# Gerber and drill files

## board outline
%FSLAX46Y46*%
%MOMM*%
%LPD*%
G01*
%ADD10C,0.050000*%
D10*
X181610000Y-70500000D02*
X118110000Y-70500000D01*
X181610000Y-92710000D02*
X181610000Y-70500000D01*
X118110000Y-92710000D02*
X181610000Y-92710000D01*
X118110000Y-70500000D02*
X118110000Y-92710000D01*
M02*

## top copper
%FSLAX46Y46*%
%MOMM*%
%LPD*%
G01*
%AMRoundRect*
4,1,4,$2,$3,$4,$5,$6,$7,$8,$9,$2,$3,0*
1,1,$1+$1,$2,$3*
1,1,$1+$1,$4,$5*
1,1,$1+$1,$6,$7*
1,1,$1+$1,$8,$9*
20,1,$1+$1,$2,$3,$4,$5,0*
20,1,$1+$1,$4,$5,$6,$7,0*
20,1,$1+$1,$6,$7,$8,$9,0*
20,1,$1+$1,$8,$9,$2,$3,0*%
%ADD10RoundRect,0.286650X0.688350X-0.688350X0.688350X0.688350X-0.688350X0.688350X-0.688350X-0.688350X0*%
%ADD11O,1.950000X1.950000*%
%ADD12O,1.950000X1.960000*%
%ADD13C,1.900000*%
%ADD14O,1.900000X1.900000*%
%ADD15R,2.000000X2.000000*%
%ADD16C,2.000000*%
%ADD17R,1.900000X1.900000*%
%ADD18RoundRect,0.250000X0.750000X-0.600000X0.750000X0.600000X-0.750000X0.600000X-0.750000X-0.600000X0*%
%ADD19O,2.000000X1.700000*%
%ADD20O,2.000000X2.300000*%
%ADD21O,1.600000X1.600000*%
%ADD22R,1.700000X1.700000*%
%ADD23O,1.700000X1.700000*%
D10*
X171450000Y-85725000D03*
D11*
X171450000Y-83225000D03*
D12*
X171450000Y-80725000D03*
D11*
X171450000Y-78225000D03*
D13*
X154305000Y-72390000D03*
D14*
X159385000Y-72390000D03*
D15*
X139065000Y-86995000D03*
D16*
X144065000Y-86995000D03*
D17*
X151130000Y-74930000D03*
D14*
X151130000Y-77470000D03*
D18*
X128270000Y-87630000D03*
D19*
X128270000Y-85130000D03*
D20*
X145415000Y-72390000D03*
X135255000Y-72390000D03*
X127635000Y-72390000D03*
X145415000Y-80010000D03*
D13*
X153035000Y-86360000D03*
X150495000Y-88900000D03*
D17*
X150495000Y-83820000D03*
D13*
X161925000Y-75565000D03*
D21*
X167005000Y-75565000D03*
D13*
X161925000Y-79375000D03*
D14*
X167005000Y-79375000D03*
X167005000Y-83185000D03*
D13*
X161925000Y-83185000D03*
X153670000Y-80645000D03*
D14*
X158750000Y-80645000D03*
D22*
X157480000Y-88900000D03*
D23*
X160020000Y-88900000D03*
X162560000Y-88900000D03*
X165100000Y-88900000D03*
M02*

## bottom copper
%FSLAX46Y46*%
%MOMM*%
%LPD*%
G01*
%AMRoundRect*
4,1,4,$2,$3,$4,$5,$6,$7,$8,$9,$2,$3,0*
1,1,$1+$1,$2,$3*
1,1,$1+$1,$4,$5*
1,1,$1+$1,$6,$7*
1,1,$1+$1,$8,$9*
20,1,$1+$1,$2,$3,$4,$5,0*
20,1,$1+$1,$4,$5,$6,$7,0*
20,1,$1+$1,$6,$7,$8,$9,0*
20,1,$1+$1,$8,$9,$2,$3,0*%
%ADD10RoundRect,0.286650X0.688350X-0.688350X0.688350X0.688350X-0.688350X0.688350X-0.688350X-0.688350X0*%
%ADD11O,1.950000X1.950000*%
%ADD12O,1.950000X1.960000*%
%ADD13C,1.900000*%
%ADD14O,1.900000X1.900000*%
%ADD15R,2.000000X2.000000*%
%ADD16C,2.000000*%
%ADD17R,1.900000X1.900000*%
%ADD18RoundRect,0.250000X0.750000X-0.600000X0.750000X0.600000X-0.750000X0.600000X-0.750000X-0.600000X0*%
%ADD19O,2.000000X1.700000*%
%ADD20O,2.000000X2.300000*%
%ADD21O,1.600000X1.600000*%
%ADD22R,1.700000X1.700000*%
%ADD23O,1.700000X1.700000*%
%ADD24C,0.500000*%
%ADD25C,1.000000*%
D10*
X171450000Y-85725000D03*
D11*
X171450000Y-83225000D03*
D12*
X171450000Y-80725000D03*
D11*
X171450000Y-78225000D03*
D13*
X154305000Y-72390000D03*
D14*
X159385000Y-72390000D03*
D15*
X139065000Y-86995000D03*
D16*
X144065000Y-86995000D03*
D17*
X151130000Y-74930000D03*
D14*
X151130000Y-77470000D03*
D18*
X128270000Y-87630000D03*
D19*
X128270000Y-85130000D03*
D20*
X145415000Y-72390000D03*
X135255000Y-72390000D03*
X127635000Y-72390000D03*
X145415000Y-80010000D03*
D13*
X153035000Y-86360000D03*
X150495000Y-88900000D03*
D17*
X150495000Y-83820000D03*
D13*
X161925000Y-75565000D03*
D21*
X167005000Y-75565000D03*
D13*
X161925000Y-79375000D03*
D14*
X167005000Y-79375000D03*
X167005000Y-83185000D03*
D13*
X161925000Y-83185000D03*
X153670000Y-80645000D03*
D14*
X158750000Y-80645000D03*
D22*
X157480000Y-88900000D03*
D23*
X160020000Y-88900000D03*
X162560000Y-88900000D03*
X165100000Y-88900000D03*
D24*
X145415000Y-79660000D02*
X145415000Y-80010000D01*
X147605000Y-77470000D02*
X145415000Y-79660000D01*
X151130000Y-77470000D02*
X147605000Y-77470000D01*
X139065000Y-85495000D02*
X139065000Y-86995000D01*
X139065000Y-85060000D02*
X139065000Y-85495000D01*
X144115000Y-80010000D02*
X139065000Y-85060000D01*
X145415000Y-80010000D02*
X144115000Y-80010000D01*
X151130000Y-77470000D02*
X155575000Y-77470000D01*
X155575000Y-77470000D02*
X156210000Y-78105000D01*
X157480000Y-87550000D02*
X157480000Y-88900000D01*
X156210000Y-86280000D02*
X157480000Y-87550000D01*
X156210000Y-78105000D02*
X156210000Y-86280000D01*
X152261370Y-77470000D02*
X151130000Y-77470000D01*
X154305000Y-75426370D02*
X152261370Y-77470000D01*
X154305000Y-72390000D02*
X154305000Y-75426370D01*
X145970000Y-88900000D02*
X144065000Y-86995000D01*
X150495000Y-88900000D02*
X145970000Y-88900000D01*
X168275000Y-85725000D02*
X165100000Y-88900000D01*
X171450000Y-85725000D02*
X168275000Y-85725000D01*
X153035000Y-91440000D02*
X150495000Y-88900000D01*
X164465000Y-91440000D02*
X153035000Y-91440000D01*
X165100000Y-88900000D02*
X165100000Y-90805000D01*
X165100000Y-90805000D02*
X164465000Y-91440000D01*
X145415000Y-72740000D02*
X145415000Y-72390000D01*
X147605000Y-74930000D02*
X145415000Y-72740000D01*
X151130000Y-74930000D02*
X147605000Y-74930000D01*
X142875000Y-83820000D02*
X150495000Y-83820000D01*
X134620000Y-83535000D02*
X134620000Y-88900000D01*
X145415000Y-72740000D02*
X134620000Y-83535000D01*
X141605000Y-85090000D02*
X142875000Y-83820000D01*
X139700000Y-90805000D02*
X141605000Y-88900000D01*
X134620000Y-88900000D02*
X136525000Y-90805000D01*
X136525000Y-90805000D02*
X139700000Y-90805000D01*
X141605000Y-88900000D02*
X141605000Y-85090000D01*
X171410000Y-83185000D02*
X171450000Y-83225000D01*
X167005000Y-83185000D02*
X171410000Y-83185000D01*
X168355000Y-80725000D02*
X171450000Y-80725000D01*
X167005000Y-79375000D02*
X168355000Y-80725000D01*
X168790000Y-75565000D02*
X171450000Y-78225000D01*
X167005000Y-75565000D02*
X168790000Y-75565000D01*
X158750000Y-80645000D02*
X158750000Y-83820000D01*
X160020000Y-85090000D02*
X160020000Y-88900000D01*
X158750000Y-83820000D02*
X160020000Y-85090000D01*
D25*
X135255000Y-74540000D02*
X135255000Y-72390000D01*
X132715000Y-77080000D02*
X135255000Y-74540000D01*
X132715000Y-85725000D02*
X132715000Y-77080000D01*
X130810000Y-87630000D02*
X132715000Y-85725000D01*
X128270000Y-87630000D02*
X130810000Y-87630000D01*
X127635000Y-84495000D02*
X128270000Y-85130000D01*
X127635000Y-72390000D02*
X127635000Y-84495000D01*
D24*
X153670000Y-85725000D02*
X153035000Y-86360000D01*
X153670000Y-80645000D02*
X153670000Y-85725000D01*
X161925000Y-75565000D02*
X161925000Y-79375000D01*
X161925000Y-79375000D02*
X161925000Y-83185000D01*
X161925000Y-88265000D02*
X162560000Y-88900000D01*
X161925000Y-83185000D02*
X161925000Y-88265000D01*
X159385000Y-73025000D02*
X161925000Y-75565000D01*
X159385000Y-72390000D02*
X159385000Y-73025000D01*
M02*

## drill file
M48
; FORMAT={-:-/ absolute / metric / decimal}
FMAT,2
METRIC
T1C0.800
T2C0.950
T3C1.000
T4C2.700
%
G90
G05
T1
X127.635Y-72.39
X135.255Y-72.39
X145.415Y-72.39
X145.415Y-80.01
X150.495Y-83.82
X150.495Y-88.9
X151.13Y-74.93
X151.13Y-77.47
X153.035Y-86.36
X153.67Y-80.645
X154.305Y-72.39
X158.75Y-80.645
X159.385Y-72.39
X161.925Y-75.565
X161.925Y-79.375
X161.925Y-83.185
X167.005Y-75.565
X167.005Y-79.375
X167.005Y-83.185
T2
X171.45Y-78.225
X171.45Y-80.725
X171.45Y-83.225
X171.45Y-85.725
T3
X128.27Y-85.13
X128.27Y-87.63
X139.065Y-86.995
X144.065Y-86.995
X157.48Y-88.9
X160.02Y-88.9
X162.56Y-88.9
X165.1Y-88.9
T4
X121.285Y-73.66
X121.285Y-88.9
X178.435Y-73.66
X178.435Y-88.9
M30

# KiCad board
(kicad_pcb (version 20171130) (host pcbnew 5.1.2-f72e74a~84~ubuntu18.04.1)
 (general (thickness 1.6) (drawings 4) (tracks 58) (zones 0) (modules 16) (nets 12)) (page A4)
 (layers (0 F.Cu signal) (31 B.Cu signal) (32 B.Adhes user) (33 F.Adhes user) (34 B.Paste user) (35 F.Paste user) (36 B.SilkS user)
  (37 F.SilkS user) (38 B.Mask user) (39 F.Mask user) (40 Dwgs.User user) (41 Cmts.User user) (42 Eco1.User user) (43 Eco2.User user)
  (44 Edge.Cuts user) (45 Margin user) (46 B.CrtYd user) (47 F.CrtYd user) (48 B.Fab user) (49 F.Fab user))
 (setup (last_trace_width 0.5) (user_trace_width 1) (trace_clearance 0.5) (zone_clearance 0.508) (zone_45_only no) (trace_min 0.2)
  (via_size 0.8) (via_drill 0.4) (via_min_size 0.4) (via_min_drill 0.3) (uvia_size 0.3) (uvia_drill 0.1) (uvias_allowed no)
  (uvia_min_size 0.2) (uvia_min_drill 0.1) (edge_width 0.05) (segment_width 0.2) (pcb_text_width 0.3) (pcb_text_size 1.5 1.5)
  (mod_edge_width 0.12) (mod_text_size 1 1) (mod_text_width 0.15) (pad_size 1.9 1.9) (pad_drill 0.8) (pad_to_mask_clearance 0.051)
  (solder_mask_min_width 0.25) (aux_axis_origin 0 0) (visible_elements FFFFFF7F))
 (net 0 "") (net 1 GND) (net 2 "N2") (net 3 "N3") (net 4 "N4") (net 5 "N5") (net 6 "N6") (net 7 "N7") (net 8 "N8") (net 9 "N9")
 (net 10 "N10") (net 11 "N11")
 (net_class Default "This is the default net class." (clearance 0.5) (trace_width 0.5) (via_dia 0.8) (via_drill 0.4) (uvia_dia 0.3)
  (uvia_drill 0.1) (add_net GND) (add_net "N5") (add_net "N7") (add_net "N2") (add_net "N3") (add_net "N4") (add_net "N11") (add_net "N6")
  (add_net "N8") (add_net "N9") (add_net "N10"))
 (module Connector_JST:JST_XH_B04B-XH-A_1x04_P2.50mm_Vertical (layer F.Cu) (at 171.45 85.725 90)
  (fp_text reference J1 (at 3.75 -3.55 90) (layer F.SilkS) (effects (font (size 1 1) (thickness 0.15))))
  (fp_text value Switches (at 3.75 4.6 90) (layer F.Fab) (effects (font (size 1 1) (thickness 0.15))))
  (pad 1 thru_hole roundrect (at 0 0 90) (size 1.95 1.95) (drill 0.95) (layers *.Cu *.Mask) (roundrect_rratio 0.147) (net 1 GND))
  (pad 2 thru_hole oval (at 2.5 0 90) (size 1.95 1.95) (drill 0.95) (layers *.Cu *.Mask) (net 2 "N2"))
  (pad 3 thru_hole oval (at 5 0 90) (size 1.96 1.95) (drill 0.95) (layers *.Cu *.Mask) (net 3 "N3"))
  (pad 4 thru_hole oval (at 7.5 0 90) (size 1.95 1.95) (drill 0.95) (layers *.Cu *.Mask) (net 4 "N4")))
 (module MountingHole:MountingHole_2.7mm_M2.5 (layer F.Cu) (at 121.285 73.66)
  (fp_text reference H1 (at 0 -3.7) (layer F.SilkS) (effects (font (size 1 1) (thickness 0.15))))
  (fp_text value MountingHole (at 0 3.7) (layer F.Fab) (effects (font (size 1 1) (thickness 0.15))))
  (pad 1 np_thru_hole circle (at 0 0) (size 2.7 2.7) (drill 2.7) (layers *.Cu *.Mask)))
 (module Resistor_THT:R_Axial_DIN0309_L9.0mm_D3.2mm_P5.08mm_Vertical (layer F.Cu) (at 154.305 72.39)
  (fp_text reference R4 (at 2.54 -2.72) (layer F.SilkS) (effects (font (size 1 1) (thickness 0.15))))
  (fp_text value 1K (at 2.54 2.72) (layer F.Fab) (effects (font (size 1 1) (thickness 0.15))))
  (pad 1 thru_hole circle (at 0 0) (size 1.9 1.9) (drill 0.8) (layers *.Cu *.Mask) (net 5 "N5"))
  (pad 2 thru_hole oval (at 5.08 0) (size 1.9 1.9) (drill 0.8) (layers *.Cu *.Mask) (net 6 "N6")))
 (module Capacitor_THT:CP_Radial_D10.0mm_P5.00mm (layer F.Cu) (at 139.065 86.995)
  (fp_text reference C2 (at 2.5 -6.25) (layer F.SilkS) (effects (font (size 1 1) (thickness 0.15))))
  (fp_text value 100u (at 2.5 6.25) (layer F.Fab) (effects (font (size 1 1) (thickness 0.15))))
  (pad 1 thru_hole rect (at 0 0) (size 2 2) (drill 1) (layers *.Cu *.Mask) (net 5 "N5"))
  (pad 2 thru_hole circle (at 5 0) (size 2 2) (drill 1) (layers *.Cu *.Mask) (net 1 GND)))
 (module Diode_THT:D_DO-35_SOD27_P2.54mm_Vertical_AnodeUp (layer F.Cu) (at 151.13 74.93 270)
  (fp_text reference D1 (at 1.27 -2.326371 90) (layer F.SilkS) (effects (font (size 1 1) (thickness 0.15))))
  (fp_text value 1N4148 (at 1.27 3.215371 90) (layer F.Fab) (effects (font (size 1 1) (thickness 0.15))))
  (pad 1 thru_hole rect (at 0 0 270) (size 1.9 1.9) (drill 0.8) (layers *.Cu *.Mask) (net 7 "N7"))
  (pad 2 thru_hole oval (at 2.54 0 270) (size 1.9 1.9) (drill 0.8) (layers *.Cu *.Mask) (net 5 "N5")))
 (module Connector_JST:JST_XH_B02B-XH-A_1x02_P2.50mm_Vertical (layer F.Cu) (at 128.27 87.63 90)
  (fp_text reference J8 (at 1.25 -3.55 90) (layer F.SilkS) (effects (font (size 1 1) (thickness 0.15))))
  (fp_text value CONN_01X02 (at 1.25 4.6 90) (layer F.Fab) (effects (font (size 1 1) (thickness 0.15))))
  (pad 1 thru_hole roundrect (at 0 0 90) (size 1.7 2) (drill 1) (layers *.Cu *.Mask) (roundrect_rratio 0.147059) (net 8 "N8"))
  (pad 2 thru_hole oval (at 2.5 0 90) (size 1.7 2) (drill 1) (layers *.Cu *.Mask) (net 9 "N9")))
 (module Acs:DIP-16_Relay (layer F.Cu) (at 145.415 72.39 270)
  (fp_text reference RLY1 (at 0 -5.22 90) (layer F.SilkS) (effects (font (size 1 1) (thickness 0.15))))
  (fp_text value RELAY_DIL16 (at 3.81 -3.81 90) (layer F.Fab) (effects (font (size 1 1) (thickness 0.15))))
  (pad 1 thru_hole oval (at 0 0 270) (size 2.3 2) (drill 0.8) (layers *.Cu *.Mask F.SilkS) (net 7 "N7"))
  (pad 5 thru_hole oval (at 0 10.16 270) (size 2.3 2) (drill 0.8) (layers *.Cu *.Mask F.SilkS) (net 8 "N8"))
  (pad 8 thru_hole oval (at 0 17.78 270) (size 2.3 2) (drill 0.8) (layers *.Cu *.Mask F.SilkS) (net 9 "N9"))
  (pad 16 thru_hole oval (at 7.62 0 270) (size 2.3 2) (drill 0.8) (layers *.Cu *.Mask F.SilkS) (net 5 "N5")))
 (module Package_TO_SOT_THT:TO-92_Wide (layer F.Cu) (at 150.495 83.82 270)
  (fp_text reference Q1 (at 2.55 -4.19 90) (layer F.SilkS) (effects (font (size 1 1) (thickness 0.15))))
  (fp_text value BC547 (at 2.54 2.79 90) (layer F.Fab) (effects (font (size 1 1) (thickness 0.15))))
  (pad 2 thru_hole circle (at 2.54 -2.54) (size 1.9 1.9) (drill 0.8) (layers *.Cu *.Mask) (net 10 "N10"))
  (pad 3 thru_hole circle (at 5.08 0) (size 1.9 1.9) (drill 0.8) (layers *.Cu *.Mask) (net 1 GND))
  (pad 1 thru_hole rect (at 0 0) (size 1.9 1.9) (drill 0.8) (layers *.Cu *.Mask) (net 7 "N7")))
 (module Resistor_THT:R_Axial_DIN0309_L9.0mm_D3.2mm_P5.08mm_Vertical (layer F.Cu) (at 161.925 75.565)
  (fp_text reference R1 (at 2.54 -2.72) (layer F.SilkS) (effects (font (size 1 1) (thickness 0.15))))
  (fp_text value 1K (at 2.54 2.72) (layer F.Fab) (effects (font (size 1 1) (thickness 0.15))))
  (pad 1 thru_hole circle (at 0 0) (size 1.9 1.9) (drill 0.8) (layers *.Cu *.Mask) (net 6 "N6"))
  (pad 2 thru_hole oval (at 5.08 0) (size 1.6 1.6) (drill 0.8) (layers *.Cu *.Mask) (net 4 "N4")))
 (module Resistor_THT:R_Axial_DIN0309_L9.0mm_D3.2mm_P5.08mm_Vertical (layer F.Cu) (at 161.925 79.375)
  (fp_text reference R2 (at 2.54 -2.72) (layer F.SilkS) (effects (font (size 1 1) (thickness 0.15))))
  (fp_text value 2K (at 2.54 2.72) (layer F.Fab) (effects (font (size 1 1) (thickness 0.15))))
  (pad 1 thru_hole circle (at 0 0) (size 1.9 1.9) (drill 0.8) (layers *.Cu *.Mask) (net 6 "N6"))
  (pad 2 thru_hole oval (at 5.08 0) (size 1.9 1.9) (drill 0.8) (layers *.Cu *.Mask) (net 3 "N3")))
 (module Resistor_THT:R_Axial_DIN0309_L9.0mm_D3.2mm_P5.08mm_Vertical (layer F.Cu) (at 161.925 83.185)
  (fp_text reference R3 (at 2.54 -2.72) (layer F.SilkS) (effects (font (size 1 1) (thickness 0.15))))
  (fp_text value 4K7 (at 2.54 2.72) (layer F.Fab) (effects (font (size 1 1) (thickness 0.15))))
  (pad 2 thru_hole oval (at 5.08 0) (size 1.9 1.9) (drill 0.8) (layers *.Cu *.Mask) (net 2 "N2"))
  (pad 1 thru_hole circle (at 0 0) (size 1.9 1.9) (drill 0.8) (layers *.Cu *.Mask) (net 6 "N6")))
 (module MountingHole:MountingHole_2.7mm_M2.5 (layer F.Cu) (at 121.285 88.9)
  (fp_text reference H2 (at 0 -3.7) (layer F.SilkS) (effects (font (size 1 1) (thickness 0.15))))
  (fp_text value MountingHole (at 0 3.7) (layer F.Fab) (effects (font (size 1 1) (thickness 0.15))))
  (pad 1 np_thru_hole circle (at 0 0) (size 2.7 2.7) (drill 2.7) (layers *.Cu *.Mask)))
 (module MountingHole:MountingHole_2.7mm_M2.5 (layer F.Cu) (at 178.435 73.66)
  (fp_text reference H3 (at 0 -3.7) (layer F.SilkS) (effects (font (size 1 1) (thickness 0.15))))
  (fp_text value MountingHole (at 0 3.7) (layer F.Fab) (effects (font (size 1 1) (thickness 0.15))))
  (pad 1 np_thru_hole circle (at 0 0) (size 2.7 2.7) (drill 2.7) (layers *.Cu *.Mask)))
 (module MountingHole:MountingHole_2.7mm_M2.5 (layer F.Cu) (at 178.435 88.9)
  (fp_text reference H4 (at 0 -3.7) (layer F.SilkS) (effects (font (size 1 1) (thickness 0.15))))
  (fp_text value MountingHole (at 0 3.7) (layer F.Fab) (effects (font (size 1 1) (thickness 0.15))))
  (pad 1 np_thru_hole circle (at 0 0) (size 2.7 2.7) (drill 2.7) (layers *.Cu *.Mask)))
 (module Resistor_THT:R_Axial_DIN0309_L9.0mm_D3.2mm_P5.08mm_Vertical (layer F.Cu) (at 153.67 80.645)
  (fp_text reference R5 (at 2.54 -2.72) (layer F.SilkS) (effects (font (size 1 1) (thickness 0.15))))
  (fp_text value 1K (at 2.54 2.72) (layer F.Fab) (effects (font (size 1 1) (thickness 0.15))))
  (pad 1 thru_hole circle (at 0 0) (size 1.9 1.9) (drill 0.8) (layers *.Cu *.Mask) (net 10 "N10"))
  (pad 2 thru_hole oval (at 5.08 0) (size 1.9 1.9) (drill 0.8) (layers *.Cu *.Mask) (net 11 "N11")))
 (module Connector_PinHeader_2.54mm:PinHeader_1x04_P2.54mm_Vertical (layer F.Cu) (at 157.48 88.9 90)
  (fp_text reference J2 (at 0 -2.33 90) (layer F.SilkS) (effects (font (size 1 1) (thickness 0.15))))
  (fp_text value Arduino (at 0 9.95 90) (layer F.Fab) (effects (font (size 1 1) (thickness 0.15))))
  (pad 1 thru_hole rect (at 0 0 90) (size 1.7 1.7) (drill 1) (layers *.Cu *.Mask) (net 5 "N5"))
  (pad 2 thru_hole oval (at 0 2.54 90) (size 1.7 1.7) (drill 1) (layers *.Cu *.Mask) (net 11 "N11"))
  (pad 3 thru_hole oval (at 0 5.08 90) (size 1.7 1.7) (drill 1) (layers *.Cu *.Mask) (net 6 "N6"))
  (pad 4 thru_hole oval (at 0 7.62 90) (size 1.7 1.7) (drill 1) (layers *.Cu *.Mask) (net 1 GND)))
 (gr_line (start 181.61 70.5) (end 118.11 70.5) (layer Edge.Cuts) (width 0.05))
 (gr_line (start 181.61 92.71) (end 181.61 70.5) (layer Edge.Cuts) (width 0.05))
 (gr_line (start 118.11 92.71) (end 181.61 92.71) (layer Edge.Cuts) (width 0.05))
 (gr_line (start 118.11 70.5) (end 118.11 92.71) (layer Edge.Cuts) (width 0.05))
 (segment (start 145.415 79.66) (end 145.415 80.01) (width 0.5) (layer B.Cu) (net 5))
 (segment (start 147.605 77.47) (end 145.415 79.66) (width 0.5) (layer B.Cu) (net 5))
 (segment (start 151.13 77.47) (end 147.605 77.47) (width 0.5) (layer B.Cu) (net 5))
 (segment (start 139.065 85.495) (end 139.065 86.995) (width 0.5) (layer B.Cu) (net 5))
 (segment (start 139.065 85.06) (end 139.065 85.495) (width 0.5) (layer B.Cu) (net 5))
 (segment (start 144.115 80.01) (end 139.065 85.06) (width 0.5) (layer B.Cu) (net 5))
 (segment (start 145.415 80.01) (end 144.115 80.01) (width 0.5) (layer B.Cu) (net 5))
 (segment (start 151.13 77.47) (end 155.575 77.47) (width 0.5) (layer B.Cu) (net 5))
 (segment (start 155.575 77.47) (end 156.21 78.105) (width 0.5) (layer B.Cu) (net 5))
 (segment (start 157.48 87.55) (end 157.48 88.9) (width 0.5) (layer B.Cu) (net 5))
 (segment (start 156.21 86.28) (end 157.48 87.55) (width 0.5) (layer B.Cu) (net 5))
 (segment (start 156.21 78.105) (end 156.21 86.28) (width 0.5) (layer B.Cu) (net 5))
 (segment (start 152.26137 77.47) (end 151.13 77.47) (width 0.5) (layer B.Cu) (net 5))
 (segment (start 154.305 75.42637) (end 152.26137 77.47) (width 0.5) (layer B.Cu) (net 5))
 (segment (start 154.305 72.39) (end 154.305 75.42637) (width 0.5) (layer B.Cu) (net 5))
 (segment (start 145.97 88.9) (end 144.065 86.995) (width 0.5) (layer B.Cu) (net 1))
 (segment (start 150.495 88.9) (end 145.97 88.9) (width 0.5) (layer B.Cu) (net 1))
 (segment (start 168.275 85.725) (end 165.1 88.9) (width 0.5) (layer B.Cu) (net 1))
 (segment (start 171.45 85.725) (end 168.275 85.725) (width 0.5) (layer B.Cu) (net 1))
 (segment (start 153.035 91.44) (end 150.495 88.9) (width 0.5) (layer B.Cu) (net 1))
 (segment (start 164.465 91.44) (end 153.035 91.44) (width 0.5) (layer B.Cu) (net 1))
 (segment (start 165.1 88.9) (end 165.1 90.805) (width 0.5) (layer B.Cu) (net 1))
 (segment (start 165.1 90.805) (end 164.465 91.44) (width 0.5) (layer B.Cu) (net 1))
 (segment (start 145.415 72.74) (end 145.415 72.39) (width 0.5) (layer B.Cu) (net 7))
 (segment (start 147.605 74.93) (end 145.415 72.74) (width 0.5) (layer B.Cu) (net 7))
 (segment (start 151.13 74.93) (end 147.605 74.93) (width 0.5) (layer B.Cu) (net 7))
 (segment (start 142.875 83.82) (end 150.495 83.82) (width 0.5) (layer B.Cu) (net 7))
 (segment (start 134.62 83.535) (end 134.62 88.9) (width 0.5) (layer B.Cu) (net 7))
 (segment (start 145.415 72.74) (end 134.62 83.535) (width 0.5) (layer B.Cu) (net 7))
 (segment (start 141.605 85.09) (end 142.875 83.82) (width 0.5) (layer B.Cu) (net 7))
 (segment (start 139.7 90.805) (end 141.605 88.9) (width 0.5) (layer B.Cu) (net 7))
 (segment (start 134.62 88.9) (end 136.525 90.805) (width 0.5) (layer B.Cu) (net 7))
 (segment (start 136.525 90.805) (end 139.7 90.805) (width 0.5) (layer B.Cu) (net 7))
 (segment (start 141.605 88.9) (end 141.605 85.09) (width 0.5) (layer B.Cu) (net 7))
 (segment (start 171.41 83.185) (end 171.45 83.225) (width 0.5) (layer B.Cu) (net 2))
 (segment (start 167.005 83.185) (end 171.41 83.185) (width 0.5) (layer B.Cu) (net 2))
 (segment (start 168.355 80.725) (end 171.45 80.725) (width 0.5) (layer B.Cu) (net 3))
 (segment (start 167.005 79.375) (end 168.355 80.725) (width 0.5) (layer B.Cu) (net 3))
 (segment (start 168.79 75.565) (end 171.45 78.225) (width 0.5) (layer B.Cu) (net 4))
 (segment (start 167.005 75.565) (end 168.79 75.565) (width 0.5) (layer B.Cu) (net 4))
 (segment (start 158.75 80.645) (end 158.75 83.82) (width 0.5) (layer B.Cu) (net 11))
 (segment (start 160.02 85.09) (end 160.02 88.9) (width 0.5) (layer B.Cu) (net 11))
 (segment (start 158.75 83.82) (end 160.02 85.09) (width 0.5) (layer B.Cu) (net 11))
 (segment (start 135.255 74.54) (end 135.255 72.39) (width 1) (layer B.Cu) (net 8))
 (segment (start 132.715 77.08) (end 135.255 74.54) (width 1) (layer B.Cu) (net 8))
 (segment (start 132.715 85.725) (end 132.715 77.08) (width 1) (layer B.Cu) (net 8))
 (segment (start 130.81 87.63) (end 132.715 85.725) (width 1) (layer B.Cu) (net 8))
 (segment (start 128.27 87.63) (end 130.81 87.63) (width 1) (layer B.Cu) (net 8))
 (segment (start 127.635 84.495) (end 128.27 85.13) (width 1) (layer B.Cu) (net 9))
 (segment (start 127.635 72.39) (end 127.635 84.495) (width 1) (layer B.Cu) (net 9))
 (segment (start 153.67 85.725) (end 153.035 86.36) (width 0.5) (layer B.Cu) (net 10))
 (segment (start 153.67 80.645) (end 153.67 85.725) (width 0.5) (layer B.Cu) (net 10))
 (segment (start 161.925 75.565) (end 161.925 79.375) (width 0.5) (layer B.Cu) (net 6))
 (segment (start 161.925 79.375) (end 161.925 83.185) (width 0.5) (layer B.Cu) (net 6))
 (segment (start 161.925 88.265) (end 162.56 88.9) (width 0.5) (layer B.Cu) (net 6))
 (segment (start 161.925 83.185) (end 161.925 88.265) (width 0.5) (layer B.Cu) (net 6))
 (segment (start 159.385 73.025) (end 161.925 75.565) (width 0.5) (layer B.Cu) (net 6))
 (segment (start 159.385 72.39) (end 159.385 73.025) (width 0.5) (layer B.Cu) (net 6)))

